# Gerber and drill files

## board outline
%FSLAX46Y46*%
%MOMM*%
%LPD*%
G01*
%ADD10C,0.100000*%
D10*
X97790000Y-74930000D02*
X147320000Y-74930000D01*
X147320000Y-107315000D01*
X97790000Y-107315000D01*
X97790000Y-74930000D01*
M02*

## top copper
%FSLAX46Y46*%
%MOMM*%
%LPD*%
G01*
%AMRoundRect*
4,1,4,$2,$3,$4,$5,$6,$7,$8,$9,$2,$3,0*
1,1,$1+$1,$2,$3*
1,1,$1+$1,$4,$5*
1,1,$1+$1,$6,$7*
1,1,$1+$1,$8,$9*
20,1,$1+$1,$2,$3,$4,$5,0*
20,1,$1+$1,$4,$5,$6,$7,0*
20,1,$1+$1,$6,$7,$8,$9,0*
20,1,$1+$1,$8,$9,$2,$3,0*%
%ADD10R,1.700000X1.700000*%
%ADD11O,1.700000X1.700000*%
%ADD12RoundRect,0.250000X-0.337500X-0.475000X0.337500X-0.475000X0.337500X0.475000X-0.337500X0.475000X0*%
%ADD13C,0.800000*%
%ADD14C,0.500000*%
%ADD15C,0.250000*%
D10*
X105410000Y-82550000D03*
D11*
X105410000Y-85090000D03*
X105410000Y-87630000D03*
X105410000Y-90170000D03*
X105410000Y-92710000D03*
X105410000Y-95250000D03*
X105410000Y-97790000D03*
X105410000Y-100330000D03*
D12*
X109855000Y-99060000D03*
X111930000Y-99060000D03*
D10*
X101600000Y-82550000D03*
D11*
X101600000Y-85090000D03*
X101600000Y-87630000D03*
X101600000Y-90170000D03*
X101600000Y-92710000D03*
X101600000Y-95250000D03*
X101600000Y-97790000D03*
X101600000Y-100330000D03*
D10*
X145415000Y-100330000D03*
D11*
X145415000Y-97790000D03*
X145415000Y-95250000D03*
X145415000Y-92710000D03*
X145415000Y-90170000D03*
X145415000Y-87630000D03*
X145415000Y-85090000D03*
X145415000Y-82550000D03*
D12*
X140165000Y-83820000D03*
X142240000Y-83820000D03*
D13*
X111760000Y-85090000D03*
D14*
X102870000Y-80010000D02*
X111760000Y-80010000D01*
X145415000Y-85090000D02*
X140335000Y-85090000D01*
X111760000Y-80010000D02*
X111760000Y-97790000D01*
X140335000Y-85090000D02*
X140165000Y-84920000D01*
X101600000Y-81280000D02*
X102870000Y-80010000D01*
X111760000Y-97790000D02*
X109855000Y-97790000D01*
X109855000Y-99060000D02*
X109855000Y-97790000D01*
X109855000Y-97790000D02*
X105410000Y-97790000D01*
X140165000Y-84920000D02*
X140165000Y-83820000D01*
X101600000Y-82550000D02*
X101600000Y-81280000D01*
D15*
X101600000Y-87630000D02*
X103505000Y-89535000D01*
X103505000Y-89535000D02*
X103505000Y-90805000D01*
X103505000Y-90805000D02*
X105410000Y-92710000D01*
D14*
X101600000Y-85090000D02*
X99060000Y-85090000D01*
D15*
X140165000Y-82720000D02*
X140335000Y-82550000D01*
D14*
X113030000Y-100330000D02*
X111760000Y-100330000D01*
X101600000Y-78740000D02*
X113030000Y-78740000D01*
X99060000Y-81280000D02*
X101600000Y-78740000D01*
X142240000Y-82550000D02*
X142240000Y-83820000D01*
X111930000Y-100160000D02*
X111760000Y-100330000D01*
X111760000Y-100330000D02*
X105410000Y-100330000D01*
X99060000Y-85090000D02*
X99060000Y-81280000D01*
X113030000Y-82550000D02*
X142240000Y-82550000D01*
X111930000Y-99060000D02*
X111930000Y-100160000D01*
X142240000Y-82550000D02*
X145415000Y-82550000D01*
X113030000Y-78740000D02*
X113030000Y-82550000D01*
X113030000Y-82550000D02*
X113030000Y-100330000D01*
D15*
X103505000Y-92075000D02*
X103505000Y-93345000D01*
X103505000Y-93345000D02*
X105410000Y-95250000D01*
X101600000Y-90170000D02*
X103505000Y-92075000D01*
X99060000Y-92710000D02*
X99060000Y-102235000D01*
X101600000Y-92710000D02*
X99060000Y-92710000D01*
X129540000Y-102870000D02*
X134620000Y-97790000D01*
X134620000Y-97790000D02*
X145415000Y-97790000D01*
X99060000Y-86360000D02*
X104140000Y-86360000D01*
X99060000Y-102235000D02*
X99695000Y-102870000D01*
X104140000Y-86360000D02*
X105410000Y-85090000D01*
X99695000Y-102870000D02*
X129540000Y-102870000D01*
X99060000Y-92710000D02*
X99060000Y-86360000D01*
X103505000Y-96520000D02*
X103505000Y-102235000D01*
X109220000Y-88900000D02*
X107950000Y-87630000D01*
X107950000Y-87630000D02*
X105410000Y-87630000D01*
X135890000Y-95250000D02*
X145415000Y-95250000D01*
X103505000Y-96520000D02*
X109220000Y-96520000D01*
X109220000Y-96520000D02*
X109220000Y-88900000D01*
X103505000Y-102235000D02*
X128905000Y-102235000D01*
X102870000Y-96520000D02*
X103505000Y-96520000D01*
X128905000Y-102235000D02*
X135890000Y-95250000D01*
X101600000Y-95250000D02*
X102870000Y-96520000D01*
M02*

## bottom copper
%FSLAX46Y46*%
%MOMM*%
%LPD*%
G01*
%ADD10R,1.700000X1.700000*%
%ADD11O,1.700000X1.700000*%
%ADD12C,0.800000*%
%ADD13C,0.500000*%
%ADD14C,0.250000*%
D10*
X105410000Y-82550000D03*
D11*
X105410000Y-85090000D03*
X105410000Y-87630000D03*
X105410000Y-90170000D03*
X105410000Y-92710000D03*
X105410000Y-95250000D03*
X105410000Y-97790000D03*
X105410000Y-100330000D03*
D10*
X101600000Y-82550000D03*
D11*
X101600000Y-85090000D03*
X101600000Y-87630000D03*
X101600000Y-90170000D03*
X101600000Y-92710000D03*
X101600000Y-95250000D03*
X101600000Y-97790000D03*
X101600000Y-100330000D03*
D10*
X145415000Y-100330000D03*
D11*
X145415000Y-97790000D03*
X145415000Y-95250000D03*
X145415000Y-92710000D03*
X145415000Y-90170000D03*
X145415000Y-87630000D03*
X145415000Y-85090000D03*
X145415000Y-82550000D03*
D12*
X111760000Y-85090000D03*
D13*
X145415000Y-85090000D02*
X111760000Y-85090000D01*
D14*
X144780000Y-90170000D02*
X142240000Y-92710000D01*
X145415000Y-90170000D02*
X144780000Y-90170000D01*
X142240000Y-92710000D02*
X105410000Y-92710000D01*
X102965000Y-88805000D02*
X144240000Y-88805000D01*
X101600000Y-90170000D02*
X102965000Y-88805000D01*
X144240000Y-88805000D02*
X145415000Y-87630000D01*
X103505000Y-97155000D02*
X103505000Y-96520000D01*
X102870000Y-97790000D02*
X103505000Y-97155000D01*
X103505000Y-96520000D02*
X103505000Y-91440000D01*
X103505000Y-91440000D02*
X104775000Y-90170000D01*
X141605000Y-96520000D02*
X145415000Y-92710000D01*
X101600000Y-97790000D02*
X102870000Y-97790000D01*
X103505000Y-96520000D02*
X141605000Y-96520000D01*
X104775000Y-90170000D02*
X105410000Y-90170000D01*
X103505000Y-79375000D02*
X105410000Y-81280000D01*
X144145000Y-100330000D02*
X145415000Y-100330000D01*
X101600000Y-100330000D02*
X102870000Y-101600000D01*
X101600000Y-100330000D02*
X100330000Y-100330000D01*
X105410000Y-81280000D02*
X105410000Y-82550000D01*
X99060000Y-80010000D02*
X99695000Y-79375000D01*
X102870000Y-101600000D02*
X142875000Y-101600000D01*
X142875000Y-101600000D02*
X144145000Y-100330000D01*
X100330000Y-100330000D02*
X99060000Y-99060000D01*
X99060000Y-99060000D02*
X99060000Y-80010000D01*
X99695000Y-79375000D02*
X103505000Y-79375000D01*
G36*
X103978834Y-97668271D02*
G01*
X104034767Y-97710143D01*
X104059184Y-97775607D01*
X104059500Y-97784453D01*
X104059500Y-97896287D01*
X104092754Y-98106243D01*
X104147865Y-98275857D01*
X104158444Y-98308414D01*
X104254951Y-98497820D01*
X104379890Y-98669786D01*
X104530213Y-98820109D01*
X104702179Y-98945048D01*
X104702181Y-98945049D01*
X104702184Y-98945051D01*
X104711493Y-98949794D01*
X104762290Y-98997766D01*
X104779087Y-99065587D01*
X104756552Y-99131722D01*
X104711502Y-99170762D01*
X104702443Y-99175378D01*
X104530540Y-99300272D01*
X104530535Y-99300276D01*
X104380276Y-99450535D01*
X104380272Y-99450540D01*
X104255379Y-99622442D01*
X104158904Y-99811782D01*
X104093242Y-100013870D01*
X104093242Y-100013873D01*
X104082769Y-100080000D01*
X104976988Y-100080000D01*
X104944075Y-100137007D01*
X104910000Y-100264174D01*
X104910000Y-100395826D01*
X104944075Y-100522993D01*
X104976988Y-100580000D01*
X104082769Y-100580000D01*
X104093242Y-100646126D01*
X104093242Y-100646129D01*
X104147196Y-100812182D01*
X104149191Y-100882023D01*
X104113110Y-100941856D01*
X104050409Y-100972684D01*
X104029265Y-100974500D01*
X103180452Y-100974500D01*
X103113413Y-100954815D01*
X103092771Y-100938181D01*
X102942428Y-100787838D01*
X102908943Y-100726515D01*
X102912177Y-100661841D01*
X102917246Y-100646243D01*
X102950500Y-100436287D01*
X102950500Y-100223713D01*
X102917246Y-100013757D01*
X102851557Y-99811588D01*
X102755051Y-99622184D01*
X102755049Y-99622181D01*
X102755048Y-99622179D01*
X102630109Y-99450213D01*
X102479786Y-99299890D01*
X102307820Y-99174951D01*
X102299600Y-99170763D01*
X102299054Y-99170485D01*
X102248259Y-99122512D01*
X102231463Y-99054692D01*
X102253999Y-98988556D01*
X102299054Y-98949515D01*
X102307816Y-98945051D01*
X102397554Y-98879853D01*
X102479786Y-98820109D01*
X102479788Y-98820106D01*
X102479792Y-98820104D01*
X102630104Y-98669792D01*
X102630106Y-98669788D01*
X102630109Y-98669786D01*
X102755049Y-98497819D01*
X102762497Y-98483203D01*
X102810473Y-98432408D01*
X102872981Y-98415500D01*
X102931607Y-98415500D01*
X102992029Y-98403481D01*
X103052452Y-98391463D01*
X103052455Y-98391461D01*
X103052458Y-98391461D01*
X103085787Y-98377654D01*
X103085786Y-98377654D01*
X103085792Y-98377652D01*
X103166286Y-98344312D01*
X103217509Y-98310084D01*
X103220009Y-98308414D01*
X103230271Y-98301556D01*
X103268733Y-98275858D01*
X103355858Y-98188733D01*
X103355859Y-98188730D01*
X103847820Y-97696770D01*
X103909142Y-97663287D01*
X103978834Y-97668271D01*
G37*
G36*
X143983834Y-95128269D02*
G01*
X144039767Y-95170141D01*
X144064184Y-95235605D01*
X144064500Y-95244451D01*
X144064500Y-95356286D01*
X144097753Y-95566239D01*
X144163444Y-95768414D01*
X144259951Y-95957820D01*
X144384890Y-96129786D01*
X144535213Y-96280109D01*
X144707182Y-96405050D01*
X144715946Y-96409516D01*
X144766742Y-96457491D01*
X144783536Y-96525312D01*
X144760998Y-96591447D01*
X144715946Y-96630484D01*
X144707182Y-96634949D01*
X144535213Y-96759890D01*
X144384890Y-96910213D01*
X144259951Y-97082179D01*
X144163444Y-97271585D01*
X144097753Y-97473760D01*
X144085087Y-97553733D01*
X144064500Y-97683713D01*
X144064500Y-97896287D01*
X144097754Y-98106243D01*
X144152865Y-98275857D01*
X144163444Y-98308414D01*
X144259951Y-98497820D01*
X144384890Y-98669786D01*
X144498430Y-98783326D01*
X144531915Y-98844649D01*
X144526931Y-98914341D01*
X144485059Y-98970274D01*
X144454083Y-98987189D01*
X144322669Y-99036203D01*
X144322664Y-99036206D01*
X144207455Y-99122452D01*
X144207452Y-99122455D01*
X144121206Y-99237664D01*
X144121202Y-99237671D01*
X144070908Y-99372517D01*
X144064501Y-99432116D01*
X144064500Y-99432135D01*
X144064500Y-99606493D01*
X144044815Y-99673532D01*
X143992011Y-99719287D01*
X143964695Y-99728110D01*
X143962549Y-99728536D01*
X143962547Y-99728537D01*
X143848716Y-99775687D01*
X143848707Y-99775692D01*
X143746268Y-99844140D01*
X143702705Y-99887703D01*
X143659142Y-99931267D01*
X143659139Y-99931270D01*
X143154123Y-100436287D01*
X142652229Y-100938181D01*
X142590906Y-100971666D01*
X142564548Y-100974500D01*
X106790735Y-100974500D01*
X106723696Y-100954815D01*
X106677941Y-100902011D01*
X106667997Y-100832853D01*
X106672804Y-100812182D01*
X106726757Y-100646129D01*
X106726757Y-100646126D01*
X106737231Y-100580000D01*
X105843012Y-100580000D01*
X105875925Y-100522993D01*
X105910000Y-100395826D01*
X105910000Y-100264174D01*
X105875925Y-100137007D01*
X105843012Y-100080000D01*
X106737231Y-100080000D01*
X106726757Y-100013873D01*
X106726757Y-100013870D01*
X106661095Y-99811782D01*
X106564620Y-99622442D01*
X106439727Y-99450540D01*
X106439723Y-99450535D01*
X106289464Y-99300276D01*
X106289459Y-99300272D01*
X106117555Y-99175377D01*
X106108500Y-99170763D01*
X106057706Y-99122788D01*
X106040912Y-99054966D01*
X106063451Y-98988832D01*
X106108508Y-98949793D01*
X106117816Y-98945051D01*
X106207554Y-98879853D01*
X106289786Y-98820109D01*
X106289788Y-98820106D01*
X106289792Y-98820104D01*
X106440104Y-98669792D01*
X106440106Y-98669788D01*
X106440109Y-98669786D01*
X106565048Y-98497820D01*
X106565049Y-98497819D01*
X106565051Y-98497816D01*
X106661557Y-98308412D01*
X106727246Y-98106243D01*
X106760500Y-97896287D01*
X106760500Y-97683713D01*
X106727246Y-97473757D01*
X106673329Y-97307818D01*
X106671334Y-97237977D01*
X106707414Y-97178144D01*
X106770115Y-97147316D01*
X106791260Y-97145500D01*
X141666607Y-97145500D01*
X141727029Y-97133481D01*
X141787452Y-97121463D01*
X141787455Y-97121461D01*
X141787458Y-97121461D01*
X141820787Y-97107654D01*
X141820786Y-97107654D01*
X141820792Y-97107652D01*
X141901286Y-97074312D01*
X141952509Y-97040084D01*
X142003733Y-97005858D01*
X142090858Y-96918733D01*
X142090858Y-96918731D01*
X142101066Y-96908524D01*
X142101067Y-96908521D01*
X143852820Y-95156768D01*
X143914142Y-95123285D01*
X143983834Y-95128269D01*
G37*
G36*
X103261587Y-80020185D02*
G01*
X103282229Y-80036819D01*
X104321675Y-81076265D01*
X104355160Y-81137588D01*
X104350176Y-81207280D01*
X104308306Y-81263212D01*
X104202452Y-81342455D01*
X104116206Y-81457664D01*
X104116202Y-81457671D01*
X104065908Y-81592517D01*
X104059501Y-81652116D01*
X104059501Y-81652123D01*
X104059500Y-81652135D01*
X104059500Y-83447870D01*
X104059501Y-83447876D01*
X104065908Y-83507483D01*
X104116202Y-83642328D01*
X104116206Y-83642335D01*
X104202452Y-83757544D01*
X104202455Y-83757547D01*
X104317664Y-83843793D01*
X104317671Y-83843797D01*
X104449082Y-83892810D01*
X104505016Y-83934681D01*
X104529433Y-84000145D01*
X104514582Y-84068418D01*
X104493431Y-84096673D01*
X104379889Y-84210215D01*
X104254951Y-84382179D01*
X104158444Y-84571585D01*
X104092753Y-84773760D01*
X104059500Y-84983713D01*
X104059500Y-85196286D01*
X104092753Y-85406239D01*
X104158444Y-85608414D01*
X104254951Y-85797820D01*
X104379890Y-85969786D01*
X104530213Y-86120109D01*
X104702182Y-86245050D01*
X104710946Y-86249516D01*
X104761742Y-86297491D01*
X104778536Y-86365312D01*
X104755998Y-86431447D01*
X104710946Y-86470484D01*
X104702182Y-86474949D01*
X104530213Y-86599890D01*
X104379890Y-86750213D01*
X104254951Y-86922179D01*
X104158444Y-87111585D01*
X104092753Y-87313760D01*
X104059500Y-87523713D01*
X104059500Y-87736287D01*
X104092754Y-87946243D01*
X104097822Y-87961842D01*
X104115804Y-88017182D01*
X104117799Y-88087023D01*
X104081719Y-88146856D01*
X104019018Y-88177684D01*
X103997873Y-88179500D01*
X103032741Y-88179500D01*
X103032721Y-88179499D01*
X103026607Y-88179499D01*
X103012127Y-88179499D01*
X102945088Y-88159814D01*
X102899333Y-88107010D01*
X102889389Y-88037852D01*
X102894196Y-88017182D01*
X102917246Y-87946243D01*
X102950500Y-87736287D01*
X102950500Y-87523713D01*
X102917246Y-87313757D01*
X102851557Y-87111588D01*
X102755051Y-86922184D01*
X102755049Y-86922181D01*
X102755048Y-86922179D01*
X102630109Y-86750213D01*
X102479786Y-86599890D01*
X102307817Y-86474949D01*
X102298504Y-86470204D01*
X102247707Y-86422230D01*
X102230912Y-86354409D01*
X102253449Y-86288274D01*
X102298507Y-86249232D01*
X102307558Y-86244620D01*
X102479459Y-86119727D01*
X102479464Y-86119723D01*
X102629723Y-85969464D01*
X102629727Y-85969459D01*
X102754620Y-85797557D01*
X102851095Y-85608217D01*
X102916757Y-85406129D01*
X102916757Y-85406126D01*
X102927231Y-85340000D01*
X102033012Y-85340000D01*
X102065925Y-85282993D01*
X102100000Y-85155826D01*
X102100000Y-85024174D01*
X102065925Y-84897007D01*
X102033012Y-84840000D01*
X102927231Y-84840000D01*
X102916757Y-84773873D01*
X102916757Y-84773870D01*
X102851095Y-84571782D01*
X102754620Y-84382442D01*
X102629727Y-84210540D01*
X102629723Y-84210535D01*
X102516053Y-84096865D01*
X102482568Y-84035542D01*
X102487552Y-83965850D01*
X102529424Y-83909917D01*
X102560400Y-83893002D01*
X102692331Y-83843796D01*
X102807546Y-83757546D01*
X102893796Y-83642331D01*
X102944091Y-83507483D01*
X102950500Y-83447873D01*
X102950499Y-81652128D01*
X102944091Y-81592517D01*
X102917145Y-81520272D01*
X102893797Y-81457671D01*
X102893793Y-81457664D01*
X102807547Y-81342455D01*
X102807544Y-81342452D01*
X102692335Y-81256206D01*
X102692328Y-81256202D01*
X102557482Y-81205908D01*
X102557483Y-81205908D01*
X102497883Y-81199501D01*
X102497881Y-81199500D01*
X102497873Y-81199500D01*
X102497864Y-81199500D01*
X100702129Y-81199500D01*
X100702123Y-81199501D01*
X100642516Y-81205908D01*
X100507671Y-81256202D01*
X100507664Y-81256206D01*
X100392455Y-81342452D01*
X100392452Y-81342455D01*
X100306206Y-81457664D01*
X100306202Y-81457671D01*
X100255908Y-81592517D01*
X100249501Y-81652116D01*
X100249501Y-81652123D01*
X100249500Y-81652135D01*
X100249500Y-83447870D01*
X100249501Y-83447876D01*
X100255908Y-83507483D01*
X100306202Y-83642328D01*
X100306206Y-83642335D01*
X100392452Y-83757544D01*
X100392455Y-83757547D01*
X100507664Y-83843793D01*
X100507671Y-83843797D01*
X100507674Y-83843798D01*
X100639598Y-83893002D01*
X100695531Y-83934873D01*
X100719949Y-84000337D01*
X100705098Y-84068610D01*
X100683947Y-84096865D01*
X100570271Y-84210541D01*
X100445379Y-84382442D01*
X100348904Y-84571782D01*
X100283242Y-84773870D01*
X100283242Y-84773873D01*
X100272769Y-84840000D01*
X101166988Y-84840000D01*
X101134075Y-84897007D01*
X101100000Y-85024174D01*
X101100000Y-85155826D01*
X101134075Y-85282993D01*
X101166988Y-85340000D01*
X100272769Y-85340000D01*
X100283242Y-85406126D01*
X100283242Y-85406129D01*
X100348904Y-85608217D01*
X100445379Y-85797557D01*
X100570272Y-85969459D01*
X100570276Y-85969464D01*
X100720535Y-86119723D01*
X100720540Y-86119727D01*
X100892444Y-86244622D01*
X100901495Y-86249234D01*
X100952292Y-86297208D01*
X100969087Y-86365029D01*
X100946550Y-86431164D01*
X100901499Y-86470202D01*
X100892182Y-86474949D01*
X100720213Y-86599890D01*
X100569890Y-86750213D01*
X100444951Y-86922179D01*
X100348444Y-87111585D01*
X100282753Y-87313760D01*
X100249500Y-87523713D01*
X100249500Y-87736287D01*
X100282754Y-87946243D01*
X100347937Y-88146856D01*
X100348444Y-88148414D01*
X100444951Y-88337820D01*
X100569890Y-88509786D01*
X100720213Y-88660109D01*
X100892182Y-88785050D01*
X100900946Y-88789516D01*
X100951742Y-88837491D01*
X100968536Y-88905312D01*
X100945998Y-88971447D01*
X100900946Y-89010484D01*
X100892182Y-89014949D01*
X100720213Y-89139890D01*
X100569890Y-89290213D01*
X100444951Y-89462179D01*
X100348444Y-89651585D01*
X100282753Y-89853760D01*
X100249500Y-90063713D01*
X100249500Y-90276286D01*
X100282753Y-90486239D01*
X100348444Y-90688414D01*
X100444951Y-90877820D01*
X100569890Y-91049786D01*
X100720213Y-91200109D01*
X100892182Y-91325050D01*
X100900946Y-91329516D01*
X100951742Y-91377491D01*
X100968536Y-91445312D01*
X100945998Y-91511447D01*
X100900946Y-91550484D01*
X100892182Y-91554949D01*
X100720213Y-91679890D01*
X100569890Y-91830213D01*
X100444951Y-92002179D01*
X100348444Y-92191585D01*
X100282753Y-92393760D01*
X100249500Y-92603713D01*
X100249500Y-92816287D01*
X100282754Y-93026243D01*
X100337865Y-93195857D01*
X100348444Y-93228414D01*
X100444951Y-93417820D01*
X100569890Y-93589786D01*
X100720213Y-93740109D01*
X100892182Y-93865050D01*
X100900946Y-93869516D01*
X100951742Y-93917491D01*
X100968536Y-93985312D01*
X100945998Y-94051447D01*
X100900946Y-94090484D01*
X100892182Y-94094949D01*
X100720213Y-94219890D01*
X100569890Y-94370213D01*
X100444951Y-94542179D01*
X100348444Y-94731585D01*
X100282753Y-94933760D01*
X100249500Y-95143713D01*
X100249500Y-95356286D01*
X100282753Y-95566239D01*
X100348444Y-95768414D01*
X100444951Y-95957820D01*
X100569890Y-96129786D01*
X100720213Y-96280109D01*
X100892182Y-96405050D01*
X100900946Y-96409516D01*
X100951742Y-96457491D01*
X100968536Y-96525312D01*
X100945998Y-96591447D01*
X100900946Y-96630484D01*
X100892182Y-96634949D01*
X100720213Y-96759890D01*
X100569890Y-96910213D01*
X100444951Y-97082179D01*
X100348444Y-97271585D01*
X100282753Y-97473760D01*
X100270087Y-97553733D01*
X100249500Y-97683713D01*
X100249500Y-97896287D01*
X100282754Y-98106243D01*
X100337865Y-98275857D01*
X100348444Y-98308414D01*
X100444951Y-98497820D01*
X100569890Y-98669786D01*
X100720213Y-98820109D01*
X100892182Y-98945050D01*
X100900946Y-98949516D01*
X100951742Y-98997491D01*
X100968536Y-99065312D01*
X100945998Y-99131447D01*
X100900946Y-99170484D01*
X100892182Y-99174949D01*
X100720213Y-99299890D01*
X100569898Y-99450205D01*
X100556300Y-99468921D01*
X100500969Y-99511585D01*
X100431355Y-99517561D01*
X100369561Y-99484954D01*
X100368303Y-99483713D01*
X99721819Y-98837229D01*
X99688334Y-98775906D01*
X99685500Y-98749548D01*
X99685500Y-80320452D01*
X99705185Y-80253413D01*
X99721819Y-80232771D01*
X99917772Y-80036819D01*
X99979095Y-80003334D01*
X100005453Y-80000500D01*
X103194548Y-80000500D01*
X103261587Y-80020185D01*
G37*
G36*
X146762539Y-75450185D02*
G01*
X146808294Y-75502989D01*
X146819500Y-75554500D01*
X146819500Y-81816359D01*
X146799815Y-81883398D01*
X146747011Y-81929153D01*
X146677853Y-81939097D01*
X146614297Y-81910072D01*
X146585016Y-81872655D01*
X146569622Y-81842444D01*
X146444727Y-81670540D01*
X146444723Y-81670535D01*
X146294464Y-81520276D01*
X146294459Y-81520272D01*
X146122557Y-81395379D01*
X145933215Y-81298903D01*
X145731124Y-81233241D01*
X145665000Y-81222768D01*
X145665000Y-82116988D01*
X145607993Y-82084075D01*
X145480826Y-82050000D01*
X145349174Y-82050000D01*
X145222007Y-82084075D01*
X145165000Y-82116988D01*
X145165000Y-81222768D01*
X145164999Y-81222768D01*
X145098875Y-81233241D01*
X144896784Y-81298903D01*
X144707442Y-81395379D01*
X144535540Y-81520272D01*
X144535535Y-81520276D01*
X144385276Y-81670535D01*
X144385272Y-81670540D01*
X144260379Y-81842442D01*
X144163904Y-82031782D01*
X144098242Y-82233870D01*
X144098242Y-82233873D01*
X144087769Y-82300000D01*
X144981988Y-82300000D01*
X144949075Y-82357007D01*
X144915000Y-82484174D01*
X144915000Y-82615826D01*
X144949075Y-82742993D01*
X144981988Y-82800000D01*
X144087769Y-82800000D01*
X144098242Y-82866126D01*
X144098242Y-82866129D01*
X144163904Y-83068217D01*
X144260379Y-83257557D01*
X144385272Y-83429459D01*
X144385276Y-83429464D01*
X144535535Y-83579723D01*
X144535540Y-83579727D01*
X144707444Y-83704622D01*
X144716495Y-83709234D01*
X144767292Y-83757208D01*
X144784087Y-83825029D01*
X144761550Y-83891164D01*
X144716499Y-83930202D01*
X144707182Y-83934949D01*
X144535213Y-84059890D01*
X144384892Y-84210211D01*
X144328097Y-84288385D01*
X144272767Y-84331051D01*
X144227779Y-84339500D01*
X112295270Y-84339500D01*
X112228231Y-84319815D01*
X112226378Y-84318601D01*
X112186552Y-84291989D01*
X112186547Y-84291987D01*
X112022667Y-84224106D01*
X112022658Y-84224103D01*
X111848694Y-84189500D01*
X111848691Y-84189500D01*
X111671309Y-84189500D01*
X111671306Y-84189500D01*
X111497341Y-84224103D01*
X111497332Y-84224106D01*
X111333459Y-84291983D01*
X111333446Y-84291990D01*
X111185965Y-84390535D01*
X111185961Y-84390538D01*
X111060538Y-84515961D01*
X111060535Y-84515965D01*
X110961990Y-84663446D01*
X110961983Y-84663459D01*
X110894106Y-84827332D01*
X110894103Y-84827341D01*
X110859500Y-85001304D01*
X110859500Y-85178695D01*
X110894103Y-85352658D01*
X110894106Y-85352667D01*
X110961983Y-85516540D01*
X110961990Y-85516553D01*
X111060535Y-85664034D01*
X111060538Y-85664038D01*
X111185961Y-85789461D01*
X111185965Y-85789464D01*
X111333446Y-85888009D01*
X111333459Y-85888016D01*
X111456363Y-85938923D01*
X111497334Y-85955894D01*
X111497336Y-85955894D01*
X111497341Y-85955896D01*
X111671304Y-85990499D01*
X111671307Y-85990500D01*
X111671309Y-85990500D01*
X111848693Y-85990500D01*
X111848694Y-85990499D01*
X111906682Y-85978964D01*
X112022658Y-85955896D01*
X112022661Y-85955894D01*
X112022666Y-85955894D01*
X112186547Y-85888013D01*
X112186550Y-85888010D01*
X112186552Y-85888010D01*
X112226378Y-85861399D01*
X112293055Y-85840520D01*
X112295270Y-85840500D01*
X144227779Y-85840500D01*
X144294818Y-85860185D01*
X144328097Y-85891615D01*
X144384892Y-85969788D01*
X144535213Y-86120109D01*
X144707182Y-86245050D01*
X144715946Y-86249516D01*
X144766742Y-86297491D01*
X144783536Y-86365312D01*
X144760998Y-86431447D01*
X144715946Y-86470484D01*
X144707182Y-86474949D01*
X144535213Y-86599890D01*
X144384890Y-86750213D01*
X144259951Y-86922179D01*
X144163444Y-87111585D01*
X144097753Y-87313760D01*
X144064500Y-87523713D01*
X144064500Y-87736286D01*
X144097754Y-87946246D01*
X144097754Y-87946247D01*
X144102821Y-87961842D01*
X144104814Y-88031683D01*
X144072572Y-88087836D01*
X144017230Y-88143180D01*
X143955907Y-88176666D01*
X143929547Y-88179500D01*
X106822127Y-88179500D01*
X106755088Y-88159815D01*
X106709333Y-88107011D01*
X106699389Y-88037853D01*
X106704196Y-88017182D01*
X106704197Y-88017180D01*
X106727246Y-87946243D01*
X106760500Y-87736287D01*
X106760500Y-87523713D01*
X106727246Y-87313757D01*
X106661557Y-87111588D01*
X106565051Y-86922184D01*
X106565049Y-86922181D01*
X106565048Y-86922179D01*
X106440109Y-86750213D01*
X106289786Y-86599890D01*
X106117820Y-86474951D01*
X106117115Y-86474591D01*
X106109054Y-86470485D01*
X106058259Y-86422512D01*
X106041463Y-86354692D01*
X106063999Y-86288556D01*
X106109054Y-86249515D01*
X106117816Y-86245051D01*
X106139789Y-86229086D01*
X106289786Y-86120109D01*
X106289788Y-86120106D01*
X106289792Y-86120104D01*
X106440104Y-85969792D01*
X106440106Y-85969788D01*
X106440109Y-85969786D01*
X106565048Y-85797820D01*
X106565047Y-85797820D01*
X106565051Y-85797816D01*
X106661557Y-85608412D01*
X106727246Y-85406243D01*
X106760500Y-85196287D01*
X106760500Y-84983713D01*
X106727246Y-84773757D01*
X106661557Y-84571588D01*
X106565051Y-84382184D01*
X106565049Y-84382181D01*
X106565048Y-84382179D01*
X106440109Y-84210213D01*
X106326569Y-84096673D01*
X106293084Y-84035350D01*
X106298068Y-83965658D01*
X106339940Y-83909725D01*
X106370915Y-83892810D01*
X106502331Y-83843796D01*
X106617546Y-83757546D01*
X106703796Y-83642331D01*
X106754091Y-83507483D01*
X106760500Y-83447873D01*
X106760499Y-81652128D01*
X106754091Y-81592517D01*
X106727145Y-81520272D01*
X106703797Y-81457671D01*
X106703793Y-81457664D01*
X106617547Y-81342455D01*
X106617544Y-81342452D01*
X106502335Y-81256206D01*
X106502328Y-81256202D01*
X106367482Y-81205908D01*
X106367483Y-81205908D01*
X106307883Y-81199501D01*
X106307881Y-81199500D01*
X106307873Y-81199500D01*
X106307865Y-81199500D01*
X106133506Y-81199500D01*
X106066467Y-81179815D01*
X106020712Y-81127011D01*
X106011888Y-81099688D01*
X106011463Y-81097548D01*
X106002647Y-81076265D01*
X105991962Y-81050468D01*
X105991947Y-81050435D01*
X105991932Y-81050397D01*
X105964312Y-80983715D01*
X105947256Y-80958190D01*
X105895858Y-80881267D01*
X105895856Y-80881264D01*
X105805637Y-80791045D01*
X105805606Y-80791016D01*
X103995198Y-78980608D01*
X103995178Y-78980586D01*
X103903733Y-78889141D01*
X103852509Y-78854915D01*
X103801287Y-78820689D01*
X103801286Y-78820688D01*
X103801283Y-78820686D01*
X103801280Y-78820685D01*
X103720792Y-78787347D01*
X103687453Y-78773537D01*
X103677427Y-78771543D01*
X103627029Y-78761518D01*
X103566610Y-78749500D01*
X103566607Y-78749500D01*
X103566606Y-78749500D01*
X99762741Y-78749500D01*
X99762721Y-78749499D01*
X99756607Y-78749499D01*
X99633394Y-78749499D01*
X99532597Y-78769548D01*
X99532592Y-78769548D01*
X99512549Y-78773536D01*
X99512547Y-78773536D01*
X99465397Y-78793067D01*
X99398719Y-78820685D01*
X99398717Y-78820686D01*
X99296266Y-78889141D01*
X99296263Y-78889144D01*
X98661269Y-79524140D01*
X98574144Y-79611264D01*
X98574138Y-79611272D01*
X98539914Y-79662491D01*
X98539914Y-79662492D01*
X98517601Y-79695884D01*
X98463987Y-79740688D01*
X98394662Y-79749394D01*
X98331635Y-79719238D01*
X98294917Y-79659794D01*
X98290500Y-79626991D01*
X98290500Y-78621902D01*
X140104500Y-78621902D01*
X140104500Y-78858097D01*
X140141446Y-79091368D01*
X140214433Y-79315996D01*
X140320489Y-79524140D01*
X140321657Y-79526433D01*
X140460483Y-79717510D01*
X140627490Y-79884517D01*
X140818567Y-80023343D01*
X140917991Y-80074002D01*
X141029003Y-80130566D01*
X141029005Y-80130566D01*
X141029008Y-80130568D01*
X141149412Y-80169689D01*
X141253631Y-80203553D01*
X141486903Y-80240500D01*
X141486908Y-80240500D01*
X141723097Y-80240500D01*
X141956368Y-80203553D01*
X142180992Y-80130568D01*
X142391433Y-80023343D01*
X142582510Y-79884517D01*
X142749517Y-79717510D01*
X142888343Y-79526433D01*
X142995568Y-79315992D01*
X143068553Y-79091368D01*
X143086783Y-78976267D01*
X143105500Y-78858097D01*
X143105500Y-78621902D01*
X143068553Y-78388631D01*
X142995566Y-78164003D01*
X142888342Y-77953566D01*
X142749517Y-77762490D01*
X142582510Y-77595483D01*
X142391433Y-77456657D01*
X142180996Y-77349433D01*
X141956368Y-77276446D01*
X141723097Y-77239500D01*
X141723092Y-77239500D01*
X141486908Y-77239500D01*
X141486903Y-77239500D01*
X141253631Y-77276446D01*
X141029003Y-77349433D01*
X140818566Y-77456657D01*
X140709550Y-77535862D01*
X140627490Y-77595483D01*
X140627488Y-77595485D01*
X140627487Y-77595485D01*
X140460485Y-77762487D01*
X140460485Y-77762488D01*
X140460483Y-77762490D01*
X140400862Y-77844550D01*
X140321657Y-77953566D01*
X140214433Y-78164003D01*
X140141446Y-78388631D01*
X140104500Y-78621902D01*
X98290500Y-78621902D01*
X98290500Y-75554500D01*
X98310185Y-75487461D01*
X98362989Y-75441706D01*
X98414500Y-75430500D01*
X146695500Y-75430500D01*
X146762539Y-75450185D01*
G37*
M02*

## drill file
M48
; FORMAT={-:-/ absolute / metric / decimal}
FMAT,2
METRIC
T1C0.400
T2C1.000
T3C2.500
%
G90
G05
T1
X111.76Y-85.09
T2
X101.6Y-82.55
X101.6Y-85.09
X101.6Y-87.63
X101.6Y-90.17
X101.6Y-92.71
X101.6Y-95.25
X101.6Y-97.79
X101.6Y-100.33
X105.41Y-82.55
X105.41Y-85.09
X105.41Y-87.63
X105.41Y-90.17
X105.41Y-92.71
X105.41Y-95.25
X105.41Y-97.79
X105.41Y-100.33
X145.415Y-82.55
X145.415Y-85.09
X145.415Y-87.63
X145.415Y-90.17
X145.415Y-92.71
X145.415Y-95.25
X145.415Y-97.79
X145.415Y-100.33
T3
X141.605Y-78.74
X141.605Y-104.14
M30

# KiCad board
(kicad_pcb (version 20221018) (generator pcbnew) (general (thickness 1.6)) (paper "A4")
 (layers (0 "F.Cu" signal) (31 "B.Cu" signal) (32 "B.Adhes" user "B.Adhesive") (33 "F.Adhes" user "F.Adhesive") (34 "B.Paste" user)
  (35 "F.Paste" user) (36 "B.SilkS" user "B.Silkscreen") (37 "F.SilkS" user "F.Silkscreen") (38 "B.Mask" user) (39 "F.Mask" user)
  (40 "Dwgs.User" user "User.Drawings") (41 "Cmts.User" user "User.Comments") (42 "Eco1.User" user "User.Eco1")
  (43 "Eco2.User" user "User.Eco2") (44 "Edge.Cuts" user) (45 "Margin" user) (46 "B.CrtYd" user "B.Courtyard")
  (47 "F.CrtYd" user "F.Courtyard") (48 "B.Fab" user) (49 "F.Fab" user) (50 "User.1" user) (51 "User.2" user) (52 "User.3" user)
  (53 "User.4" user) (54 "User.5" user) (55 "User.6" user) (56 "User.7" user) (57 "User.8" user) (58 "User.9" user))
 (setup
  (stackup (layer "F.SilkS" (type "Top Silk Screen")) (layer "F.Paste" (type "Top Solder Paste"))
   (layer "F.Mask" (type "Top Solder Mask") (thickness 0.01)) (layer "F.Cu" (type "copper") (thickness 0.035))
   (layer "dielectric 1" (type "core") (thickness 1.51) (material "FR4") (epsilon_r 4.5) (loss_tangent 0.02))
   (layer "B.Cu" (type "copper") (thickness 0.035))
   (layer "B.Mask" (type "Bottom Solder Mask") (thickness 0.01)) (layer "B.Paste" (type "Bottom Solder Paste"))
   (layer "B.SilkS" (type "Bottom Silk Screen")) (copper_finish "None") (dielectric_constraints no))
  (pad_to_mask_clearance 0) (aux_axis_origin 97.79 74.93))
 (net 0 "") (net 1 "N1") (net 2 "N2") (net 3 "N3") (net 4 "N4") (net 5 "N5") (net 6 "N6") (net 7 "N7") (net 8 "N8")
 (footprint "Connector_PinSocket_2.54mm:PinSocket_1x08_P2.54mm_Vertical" (layer "F.Cu") (at 105.41 82.55)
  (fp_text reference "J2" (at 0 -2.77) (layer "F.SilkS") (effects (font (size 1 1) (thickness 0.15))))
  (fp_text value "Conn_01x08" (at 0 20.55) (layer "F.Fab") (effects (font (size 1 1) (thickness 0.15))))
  (pad "1" thru_hole rect (at 0 0) (size 1.7 1.7) (drill 1) (layers "*.Cu" "*.Mask") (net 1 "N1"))
  (pad "2" thru_hole oval (at 0 2.54) (size 1.7 1.7) (drill 1) (layers "*.Cu" "*.Mask") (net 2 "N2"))
  (pad "3" thru_hole oval (at 0 5.08) (size 1.7 1.7) (drill 1) (layers "*.Cu" "*.Mask") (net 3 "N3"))
  (pad "4" thru_hole oval (at 0 7.62) (size 1.7 1.7) (drill 1) (layers "*.Cu" "*.Mask") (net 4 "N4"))
  (pad "5" thru_hole oval (at 0 10.16) (size 1.7 1.7) (drill 1) (layers "*.Cu" "*.Mask") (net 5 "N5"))
  (pad "6" thru_hole oval (at 0 12.7) (size 1.7 1.7) (drill 1) (layers "*.Cu" "*.Mask") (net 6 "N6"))
  (pad "7" thru_hole oval (at 0 15.24) (size 1.7 1.7) (drill 1) (layers "*.Cu" "*.Mask") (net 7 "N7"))
  (pad "8" thru_hole oval (at 0 17.78) (size 1.7 1.7) (drill 1) (layers "*.Cu" "*.Mask") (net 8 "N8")))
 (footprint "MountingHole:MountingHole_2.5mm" (layer "F.Cu") (at 141.605 104.14)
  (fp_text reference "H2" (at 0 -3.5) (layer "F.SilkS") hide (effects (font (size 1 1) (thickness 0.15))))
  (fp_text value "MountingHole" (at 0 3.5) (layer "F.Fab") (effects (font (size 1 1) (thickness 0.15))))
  (pad "" np_thru_hole circle (at 0 0) (size 2.5 2.5) (drill 2.5) (layers "*.Cu" "*.Mask")))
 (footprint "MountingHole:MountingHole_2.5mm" (layer "F.Cu") (at 141.605 78.74)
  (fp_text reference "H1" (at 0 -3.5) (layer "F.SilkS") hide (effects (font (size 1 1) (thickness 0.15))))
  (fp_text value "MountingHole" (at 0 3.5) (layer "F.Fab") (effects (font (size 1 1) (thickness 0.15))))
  (pad "" np_thru_hole circle (at 0 0) (size 2.5 2.5) (drill 2.5) (layers "*.Cu" "*.Mask")))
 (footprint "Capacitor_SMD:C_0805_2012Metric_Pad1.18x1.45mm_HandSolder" (layer "F.Cu") (at 110.8925 99.06)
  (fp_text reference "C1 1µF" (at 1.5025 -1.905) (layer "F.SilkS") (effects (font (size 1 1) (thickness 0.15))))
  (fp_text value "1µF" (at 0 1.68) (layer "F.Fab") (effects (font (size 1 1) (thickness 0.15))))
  (pad "1" smd roundrect (at -1.0375 0) (size 1.175 1.45) (layers "F.Cu" "F.Paste" "F.Mask") (roundrect_rratio 0.2127659574) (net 7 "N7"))
  (pad "2" smd roundrect (at 1.0375 0) (size 1.175 1.45) (layers "F.Cu" "F.Paste" "F.Mask") (roundrect_rratio 0.2127659574) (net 8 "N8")))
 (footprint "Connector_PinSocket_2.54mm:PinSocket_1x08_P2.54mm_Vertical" (layer "F.Cu") (at 101.6 82.55)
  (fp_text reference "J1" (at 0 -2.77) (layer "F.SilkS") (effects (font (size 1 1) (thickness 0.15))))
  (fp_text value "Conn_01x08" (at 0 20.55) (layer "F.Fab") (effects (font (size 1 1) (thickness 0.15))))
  (pad "1" thru_hole rect (at 0 0) (size 1.7 1.7) (drill 1) (layers "*.Cu" "*.Mask") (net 7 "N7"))
  (pad "2" thru_hole oval (at 0 2.54) (size 1.7 1.7) (drill 1) (layers "*.Cu" "*.Mask") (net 8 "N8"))
  (pad "3" thru_hole oval (at 0 5.08) (size 1.7 1.7) (drill 1) (layers "*.Cu" "*.Mask") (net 5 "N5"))
  (pad "4" thru_hole oval (at 0 7.62) (size 1.7 1.7) (drill 1) (layers "*.Cu" "*.Mask") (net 6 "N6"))
  (pad "5" thru_hole oval (at 0 10.16) (size 1.7 1.7) (drill 1) (layers "*.Cu" "*.Mask") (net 2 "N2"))
  (pad "6" thru_hole oval (at 0 12.7) (size 1.7 1.7) (drill 1) (layers "*.Cu" "*.Mask") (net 3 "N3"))
  (pad "7" thru_hole oval (at 0 15.24) (size 1.7 1.7) (drill 1) (layers "*.Cu" "*.Mask") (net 4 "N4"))
  (pad "8" thru_hole oval (at 0 17.78) (size 1.7 1.7) (drill 1) (layers "*.Cu" "*.Mask") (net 1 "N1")))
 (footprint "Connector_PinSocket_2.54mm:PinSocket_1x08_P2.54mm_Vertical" (layer "F.Cu") (at 145.415 100.33 180)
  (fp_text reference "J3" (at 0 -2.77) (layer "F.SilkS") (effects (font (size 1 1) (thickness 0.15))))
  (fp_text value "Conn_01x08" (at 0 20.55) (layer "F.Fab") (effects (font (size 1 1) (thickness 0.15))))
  (pad "1" thru_hole rect (at 0 0 180) (size 1.7 1.7) (drill 1) (layers "*.Cu" "*.Mask") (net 1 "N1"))
  (pad "2" thru_hole oval (at 0 2.54 180) (size 1.7 1.7) (drill 1) (layers "*.Cu" "*.Mask") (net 2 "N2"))
  (pad "3" thru_hole oval (at 0 5.08 180) (size 1.7 1.7) (drill 1) (layers "*.Cu" "*.Mask") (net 3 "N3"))
  (pad "4" thru_hole oval (at 0 7.62 180) (size 1.7 1.7) (drill 1) (layers "*.Cu" "*.Mask") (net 4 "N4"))
  (pad "5" thru_hole oval (at 0 10.16 180) (size 1.7 1.7) (drill 1) (layers "*.Cu" "*.Mask") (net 5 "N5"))
  (pad "6" thru_hole oval (at 0 12.7 180) (size 1.7 1.7) (drill 1) (layers "*.Cu" "*.Mask") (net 6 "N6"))
  (pad "7" thru_hole oval (at 0 15.24 180) (size 1.7 1.7) (drill 1) (layers "*.Cu" "*.Mask") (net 7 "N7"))
  (pad "8" thru_hole oval (at 0 17.78 180) (size 1.7 1.7) (drill 1) (layers "*.Cu" "*.Mask") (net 8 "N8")))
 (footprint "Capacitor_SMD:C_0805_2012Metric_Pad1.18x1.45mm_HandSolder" (layer "F.Cu") (at 141.2025 83.82)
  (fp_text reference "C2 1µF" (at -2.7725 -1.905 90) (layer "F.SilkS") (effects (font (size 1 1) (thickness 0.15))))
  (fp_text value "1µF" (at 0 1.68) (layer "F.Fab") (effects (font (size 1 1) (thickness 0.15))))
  (pad "1" smd roundrect (at -1.0375 0) (size 1.175 1.45) (layers "F.Cu" "F.Paste" "F.Mask") (roundrect_rratio 0.2127659574) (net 7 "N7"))
  (pad "2" smd roundrect (at 1.0375 0) (size 1.175 1.45) (layers "F.Cu" "F.Paste" "F.Mask") (roundrect_rratio 0.2127659574) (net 8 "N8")))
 (gr_rect (start 97.79 74.93) (end 147.32 107.315) (stroke (width 0.1) (type default)) (fill none) (layer "Edge.Cuts"))
 (segment (start 102.87 80.01) (end 111.76 80.01) (width 0.5) (layer "F.Cu") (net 7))
 (segment (start 145.415 85.09) (end 140.335 85.09) (width 0.5) (layer "F.Cu") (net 7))
 (segment (start 111.76 80.01) (end 111.76 97.79) (width 0.5) (layer "F.Cu") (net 7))
 (segment (start 140.335 85.09) (end 140.165 84.92) (width 0.5) (layer "F.Cu") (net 7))
 (segment (start 101.6 81.28) (end 102.87 80.01) (width 0.5) (layer "F.Cu") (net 7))
 (segment (start 111.76 97.79) (end 109.855 97.79) (width 0.5) (layer "F.Cu") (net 7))
 (segment (start 109.855 99.06) (end 109.855 97.79) (width 0.5) (layer "F.Cu") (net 7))
 (segment (start 109.855 97.79) (end 105.41 97.79) (width 0.5) (layer "F.Cu") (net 7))
 (segment (start 140.165 84.92) (end 140.165 83.82) (width 0.5) (layer "F.Cu") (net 7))
 (segment (start 101.6 82.55) (end 101.6 81.28) (width 0.5) (layer "F.Cu") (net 7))
 (via (at 111.76 85.09) (size 0.8) (drill 0.4) (layers "F.Cu" "B.Cu") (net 7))
 (segment (start 145.415 85.09) (end 111.76 85.09) (width 0.5) (layer "B.Cu") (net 7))
 (segment (start 101.6 87.63) (end 103.505 89.535) (width 0.25) (layer "F.Cu") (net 5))
 (segment (start 103.505 89.535) (end 103.505 90.805) (width 0.25) (layer "F.Cu") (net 5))
 (segment (start 103.505 90.805) (end 105.41 92.71) (width 0.25) (layer "F.Cu") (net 5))
 (segment (start 144.78 90.17) (end 142.24 92.71) (width 0.25) (layer "B.Cu") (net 5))
 (segment (start 145.415 90.17) (end 144.78 90.17) (width 0.25) (layer "B.Cu") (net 5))
 (segment (start 142.24 92.71) (end 105.41 92.71) (width 0.25) (layer "B.Cu") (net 5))
 (segment (start 101.6 85.09) (end 99.06 85.09) (width 0.5) (layer "F.Cu") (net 8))
 (segment (start 140.165 82.72) (end 140.335 82.55) (width 0.25) (layer "F.Cu") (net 8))
 (segment (start 113.03 100.33) (end 111.76 100.33) (width 0.5) (layer "F.Cu") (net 8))
 (segment (start 101.6 78.74) (end 113.03 78.74) (width 0.5) (layer "F.Cu") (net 8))
 (segment (start 99.06 81.28) (end 101.6 78.74) (width 0.5) (layer "F.Cu") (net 8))
 (segment (start 142.24 82.55) (end 142.24 83.82) (width 0.5) (layer "F.Cu") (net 8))
 (segment (start 111.93 100.16) (end 111.76 100.33) (width 0.5) (layer "F.Cu") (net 8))
 (segment (start 111.76 100.33) (end 105.41 100.33) (width 0.5) (layer "F.Cu") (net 8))
 (segment (start 99.06 85.09) (end 99.06 81.28) (width 0.5) (layer "F.Cu") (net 8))
 (segment (start 113.03 82.55) (end 142.24 82.55) (width 0.5) (layer "F.Cu") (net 8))
 (segment (start 111.93 99.06) (end 111.93 100.16) (width 0.5) (layer "F.Cu") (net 8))
 (segment (start 142.24 82.55) (end 145.415 82.55) (width 0.5) (layer "F.Cu") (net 8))
 (segment (start 113.03 78.74) (end 113.03 82.55) (width 0.5) (layer "F.Cu") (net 8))
 (segment (start 113.03 82.55) (end 113.03 100.33) (width 0.5) (layer "F.Cu") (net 8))
 (segment (start 103.505 92.075) (end 103.505 93.345) (width 0.25) (layer "F.Cu") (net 6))
 (segment (start 103.505 93.345) (end 105.41 95.25) (width 0.25) (layer "F.Cu") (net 6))
 (segment (start 101.6 90.17) (end 103.505 92.075) (width 0.25) (layer "F.Cu") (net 6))
 (segment (start 102.965 88.805) (end 144.24 88.805) (width 0.25) (layer "B.Cu") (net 6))
 (segment (start 101.6 90.17) (end 102.965 88.805) (width 0.25) (layer "B.Cu") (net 6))
 (segment (start 144.24 88.805) (end 145.415 87.63) (width 0.25) (layer "B.Cu") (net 6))
 (segment (start 99.06 92.71) (end 99.06 102.235) (width 0.25) (layer "F.Cu") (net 2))
 (segment (start 101.6 92.71) (end 99.06 92.71) (width 0.25) (layer "F.Cu") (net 2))
 (segment (start 129.54 102.87) (end 134.62 97.79) (width 0.25) (layer "F.Cu") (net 2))
 (segment (start 134.62 97.79) (end 145.415 97.79) (width 0.25) (layer "F.Cu") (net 2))
 (segment (start 99.06 86.36) (end 104.14 86.36) (width 0.25) (layer "F.Cu") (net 2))
 (segment (start 99.06 102.235) (end 99.695 102.87) (width 0.25) (layer "F.Cu") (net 2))
 (segment (start 104.14 86.36) (end 105.41 85.09) (width 0.25) (layer "F.Cu") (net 2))
 (segment (start 99.695 102.87) (end 129.54 102.87) (width 0.25) (layer "F.Cu") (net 2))
 (segment (start 99.06 92.71) (end 99.06 86.36) (width 0.25) (layer "F.Cu") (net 2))
 (segment (start 103.505 96.52) (end 103.505 102.235) (width 0.25) (layer "F.Cu") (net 3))
 (segment (start 109.22 88.9) (end 107.95 87.63) (width 0.25) (layer "F.Cu") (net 3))
 (segment (start 107.95 87.63) (end 105.41 87.63) (width 0.25) (layer "F.Cu") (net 3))
 (segment (start 135.89 95.25) (end 145.415 95.25) (width 0.25) (layer "F.Cu") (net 3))
 (segment (start 103.505 96.52) (end 109.22 96.52) (width 0.25) (layer "F.Cu") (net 3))
 (segment (start 109.22 96.52) (end 109.22 88.9) (width 0.25) (layer "F.Cu") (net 3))
 (segment (start 103.505 102.235) (end 128.905 102.235) (width 0.25) (layer "F.Cu") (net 3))
 (segment (start 102.87 96.52) (end 103.505 96.52) (width 0.25) (layer "F.Cu") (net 3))
 (segment (start 128.905 102.235) (end 135.89 95.25) (width 0.25) (layer "F.Cu") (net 3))
 (segment (start 101.6 95.25) (end 102.87 96.52) (width 0.25) (layer "F.Cu") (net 3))
 (segment (start 103.505 97.155) (end 103.505 96.52) (width 0.25) (layer "B.Cu") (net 4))
 (segment (start 102.87 97.79) (end 103.505 97.155) (width 0.25) (layer "B.Cu") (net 4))
 (segment (start 103.505 96.52) (end 103.505 91.44) (width 0.25) (layer "B.Cu") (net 4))
 (segment (start 103.505 91.44) (end 104.775 90.17) (width 0.25) (layer "B.Cu") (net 4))
 (segment (start 141.605 96.52) (end 145.415 92.71) (width 0.25) (layer "B.Cu") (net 4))
 (segment (start 101.6 97.79) (end 102.87 97.79) (width 0.25) (layer "B.Cu") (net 4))
 (segment (start 103.505 96.52) (end 141.605 96.52) (width 0.25) (layer "B.Cu") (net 4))
 (segment (start 104.775 90.17) (end 105.41 90.17) (width 0.25) (layer "B.Cu") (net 4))
 (segment (start 103.505 79.375) (end 105.41 81.28) (width 0.25) (layer "B.Cu") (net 1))
 (segment (start 144.145 100.33) (end 145.415 100.33) (width 0.25) (layer "B.Cu") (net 1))
 (segment (start 101.6 100.33) (end 102.87 101.6) (width 0.25) (layer "B.Cu") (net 1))
 (segment (start 101.6 100.33) (end 100.33 100.33) (width 0.25) (layer "B.Cu") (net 1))
 (segment (start 105.41 81.28) (end 105.41 82.55) (width 0.25) (layer "B.Cu") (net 1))
 (segment (start 99.06 80.01) (end 99.695 79.375) (width 0.25) (layer "B.Cu") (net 1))
 (segment (start 102.87 101.6) (end 142.875 101.6) (width 0.25) (layer "B.Cu") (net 1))
 (segment (start 142.875 101.6) (end 144.145 100.33) (width 0.25) (layer "B.Cu") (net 1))
 (segment (start 100.33 100.33) (end 99.06 99.06) (width 0.25) (layer "B.Cu") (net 1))
 (segment (start 99.06 99.06) (end 99.06 80.01) (width 0.25) (layer "B.Cu") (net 1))
 (segment (start 99.695 79.375) (end 103.505 79.375) (width 0.25) (layer "B.Cu") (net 1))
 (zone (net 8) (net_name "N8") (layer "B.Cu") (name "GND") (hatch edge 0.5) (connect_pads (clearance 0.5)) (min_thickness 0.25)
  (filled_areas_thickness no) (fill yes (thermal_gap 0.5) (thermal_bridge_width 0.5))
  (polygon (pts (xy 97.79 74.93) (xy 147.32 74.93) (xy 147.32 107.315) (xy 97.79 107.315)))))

